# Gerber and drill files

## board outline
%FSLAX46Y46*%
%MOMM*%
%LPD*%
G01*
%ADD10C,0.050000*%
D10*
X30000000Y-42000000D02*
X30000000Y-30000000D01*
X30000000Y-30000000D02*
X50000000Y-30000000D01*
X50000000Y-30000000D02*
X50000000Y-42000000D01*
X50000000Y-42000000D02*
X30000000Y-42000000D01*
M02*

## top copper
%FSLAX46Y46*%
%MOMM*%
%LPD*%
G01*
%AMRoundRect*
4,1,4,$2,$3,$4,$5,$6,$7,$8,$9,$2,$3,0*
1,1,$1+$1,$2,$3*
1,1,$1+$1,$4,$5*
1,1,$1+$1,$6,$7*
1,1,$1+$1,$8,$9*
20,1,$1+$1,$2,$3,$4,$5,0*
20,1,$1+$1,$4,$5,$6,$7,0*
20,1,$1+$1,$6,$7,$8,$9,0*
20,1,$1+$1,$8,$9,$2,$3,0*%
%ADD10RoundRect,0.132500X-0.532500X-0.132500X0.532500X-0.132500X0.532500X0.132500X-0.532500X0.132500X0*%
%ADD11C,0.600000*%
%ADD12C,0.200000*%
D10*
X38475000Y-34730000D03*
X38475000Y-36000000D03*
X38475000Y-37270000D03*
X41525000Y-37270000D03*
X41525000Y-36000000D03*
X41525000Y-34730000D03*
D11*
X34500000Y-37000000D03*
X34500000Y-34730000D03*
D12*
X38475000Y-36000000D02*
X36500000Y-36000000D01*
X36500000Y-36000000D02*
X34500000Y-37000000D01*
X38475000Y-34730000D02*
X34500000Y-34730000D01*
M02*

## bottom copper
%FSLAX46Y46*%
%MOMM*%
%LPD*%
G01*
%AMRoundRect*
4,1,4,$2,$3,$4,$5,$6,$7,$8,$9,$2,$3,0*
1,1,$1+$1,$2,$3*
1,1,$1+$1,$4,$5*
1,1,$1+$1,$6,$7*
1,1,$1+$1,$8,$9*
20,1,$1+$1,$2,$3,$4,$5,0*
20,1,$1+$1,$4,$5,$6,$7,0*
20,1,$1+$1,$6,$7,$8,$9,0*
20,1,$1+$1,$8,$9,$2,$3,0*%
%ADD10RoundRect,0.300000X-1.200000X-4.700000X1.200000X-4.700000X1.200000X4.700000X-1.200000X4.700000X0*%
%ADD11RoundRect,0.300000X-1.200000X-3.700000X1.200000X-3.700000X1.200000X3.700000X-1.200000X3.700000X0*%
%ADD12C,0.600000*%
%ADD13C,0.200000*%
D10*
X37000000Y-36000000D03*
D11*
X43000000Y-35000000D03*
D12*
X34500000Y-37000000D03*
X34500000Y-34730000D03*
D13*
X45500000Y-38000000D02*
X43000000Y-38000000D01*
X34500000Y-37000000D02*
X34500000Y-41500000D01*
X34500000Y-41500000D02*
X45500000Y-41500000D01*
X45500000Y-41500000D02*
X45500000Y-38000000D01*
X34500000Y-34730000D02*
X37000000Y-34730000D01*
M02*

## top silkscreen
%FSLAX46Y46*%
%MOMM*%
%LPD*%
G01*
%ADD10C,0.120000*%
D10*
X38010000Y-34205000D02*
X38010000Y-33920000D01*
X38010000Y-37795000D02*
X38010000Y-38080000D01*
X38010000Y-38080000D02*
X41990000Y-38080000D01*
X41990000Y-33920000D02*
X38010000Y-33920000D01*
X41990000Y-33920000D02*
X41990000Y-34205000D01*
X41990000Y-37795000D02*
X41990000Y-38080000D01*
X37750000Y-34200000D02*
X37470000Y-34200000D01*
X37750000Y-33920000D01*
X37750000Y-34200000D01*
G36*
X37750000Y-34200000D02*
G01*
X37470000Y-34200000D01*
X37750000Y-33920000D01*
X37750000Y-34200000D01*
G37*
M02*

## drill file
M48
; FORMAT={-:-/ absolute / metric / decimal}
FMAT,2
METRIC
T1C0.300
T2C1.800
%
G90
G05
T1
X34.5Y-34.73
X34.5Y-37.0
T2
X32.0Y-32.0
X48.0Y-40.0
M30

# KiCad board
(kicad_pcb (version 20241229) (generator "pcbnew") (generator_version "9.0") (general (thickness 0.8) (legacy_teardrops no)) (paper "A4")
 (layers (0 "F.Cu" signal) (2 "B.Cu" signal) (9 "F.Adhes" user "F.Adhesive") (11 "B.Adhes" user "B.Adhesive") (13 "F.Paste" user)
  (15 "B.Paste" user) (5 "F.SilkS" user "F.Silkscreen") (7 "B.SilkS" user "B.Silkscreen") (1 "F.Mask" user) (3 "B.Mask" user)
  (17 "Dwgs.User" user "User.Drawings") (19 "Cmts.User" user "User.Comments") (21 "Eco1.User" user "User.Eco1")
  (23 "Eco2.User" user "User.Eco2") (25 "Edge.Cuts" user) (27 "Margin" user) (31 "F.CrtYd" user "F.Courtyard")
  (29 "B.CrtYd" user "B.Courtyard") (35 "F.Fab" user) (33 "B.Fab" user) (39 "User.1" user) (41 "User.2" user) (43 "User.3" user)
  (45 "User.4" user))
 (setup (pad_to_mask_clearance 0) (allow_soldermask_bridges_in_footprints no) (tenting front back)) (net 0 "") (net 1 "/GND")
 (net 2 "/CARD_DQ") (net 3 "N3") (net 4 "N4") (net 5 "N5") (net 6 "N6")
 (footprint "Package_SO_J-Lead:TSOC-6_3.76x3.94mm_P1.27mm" (layer "F.Cu") (at 40 36)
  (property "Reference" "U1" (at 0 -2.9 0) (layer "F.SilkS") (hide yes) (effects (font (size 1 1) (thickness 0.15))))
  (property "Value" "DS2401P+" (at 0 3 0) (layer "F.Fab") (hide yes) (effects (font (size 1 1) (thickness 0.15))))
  (fp_line (start -1.99 -1.795) (end -1.99 -2.08) (stroke (width 0.12) (type solid)) (layer "F.SilkS"))
  (fp_line (start -1.99 1.795) (end -1.99 2.08) (stroke (width 0.12) (type solid)) (layer "F.SilkS"))
  (fp_line (start -1.99 2.08) (end 1.99 2.08) (stroke (width 0.12) (type solid)) (layer "F.SilkS"))
  (fp_line (start 1.99 -2.08) (end -1.99 -2.08) (stroke (width 0.12) (type solid)) (layer "F.SilkS"))
  (fp_line (start 1.99 -2.08) (end 1.99 -1.795) (stroke (width 0.12) (type solid)) (layer "F.SilkS"))
  (fp_line (start 1.99 1.795) (end 1.99 2.08) (stroke (width 0.12) (type solid)) (layer "F.SilkS"))
  (fp_poly
   (pts (xy -2.25 -1.8) (xy -2.53 -1.8) (xy -2.25 -2.08) (xy -2.25 -1.8)) (stroke (width 0.12) (type solid)) (fill yes) (layer "F.SilkS"))
  (pad "1" smd roundrect (at -1.525 -1.27) (size 1.33 0.53) (layers "F.Cu" "F.Mask" "F.Paste") (roundrect_rratio 0.25) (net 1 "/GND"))
  (pad "2" smd roundrect (at -1.525 0) (size 1.33 0.53) (layers "F.Cu" "F.Mask" "F.Paste") (roundrect_rratio 0.25) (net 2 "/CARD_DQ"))
  (pad "3" smd roundrect (at -1.525 1.27) (size 1.33 0.53) (layers "F.Cu" "F.Mask" "F.Paste") (roundrect_rratio 0.25) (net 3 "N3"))
  (pad "4" smd roundrect (at 1.525 1.27) (size 1.33 0.53) (layers "F.Cu" "F.Mask" "F.Paste") (roundrect_rratio 0.25) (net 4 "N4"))
  (pad "5" smd roundrect (at 1.525 0) (size 1.33 0.53) (layers "F.Cu" "F.Mask" "F.Paste") (roundrect_rratio 0.25) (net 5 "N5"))
  (pad "6" smd roundrect (at 1.525 -1.27) (size 1.33 0.53) (layers "F.Cu" "F.Mask" "F.Paste") (roundrect_rratio 0.25) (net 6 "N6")))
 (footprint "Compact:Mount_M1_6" (layer "F.Cu") (at 32 32)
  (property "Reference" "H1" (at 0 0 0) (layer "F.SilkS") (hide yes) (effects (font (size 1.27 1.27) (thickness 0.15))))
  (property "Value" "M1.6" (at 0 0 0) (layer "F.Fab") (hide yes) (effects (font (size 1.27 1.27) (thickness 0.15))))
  (pad "" np_thru_hole circle (at 0 0) (size 1.8 1.8) (drill 1.8) (layers "*.Cu")))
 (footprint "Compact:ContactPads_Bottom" (layer "F.Cu") (at 30 30)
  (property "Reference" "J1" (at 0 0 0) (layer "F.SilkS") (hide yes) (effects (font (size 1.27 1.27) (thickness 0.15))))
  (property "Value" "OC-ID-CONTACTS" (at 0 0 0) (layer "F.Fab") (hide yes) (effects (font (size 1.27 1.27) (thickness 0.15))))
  (pad "1" smd roundrect (at 7 6) (size 3 10) (layers "B.Cu" "B.Mask") (roundrect_rratio 0.1) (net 1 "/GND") (thermal_bridge_angle 45))
  (pad "2" smd roundrect (at 13 5) (size 3 8) (layers "B.Cu" "B.Mask") (roundrect_rratio 0.1) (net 2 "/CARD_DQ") (thermal_bridge_angle 45)))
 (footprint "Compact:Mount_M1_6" (layer "F.Cu") (at 48 40)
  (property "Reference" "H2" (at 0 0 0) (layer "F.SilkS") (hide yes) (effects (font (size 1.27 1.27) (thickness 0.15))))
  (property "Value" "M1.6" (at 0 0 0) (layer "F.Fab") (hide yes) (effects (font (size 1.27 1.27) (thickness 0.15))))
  (pad "" np_thru_hole circle (at 0 0) (size 1.8 1.8) (drill 1.8) (layers "*.Cu")))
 (gr_line (start 30 42) (end 30 30) (stroke (width 0.05) (type default)) (layer "Edge.Cuts"))
 (gr_line (start 30 30) (end 50 30) (stroke (width 0.05) (type default)) (layer "Edge.Cuts"))
 (gr_line (start 50 30) (end 50 42) (stroke (width 0.05) (type default)) (layer "Edge.Cuts"))
 (gr_line (start 50 42) (end 30 42) (stroke (width 0.05) (type default)) (layer "Edge.Cuts"))
 (segment (start 38.475 36) (end 36.5 36) (width 0.2) (layer "F.Cu") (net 2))
 (segment (start 36.5 36) (end 34.5 37) (width 0.2) (layer "F.Cu") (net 2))
 (via (at 34.5 37) (size 0.6) (drill 0.3) (layers "F.Cu" "B.Cu") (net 2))
 (segment (start 45.5 38) (end 43 38) (width 0.2) (layer "B.Cu") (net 2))
 (segment (start 34.5 37) (end 34.5 41.5) (width 0.2) (layer "B.Cu") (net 2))
 (segment (start 34.5 41.5) (end 45.5 41.5) (width 0.2) (layer "B.Cu") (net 2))
 (segment (start 45.5 41.5) (end 45.5 38) (width 0.2) (layer "B.Cu") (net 2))
 (segment (start 38.475 34.73) (end 34.5 34.73) (width 0.2) (layer "F.Cu") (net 1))
 (via (at 34.5 34.73) (size 0.6) (drill 0.3) (layers "F.Cu" "B.Cu") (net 1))
 (segment (start 34.5 34.73) (end 37 34.73) (width 0.2) (layer "B.Cu") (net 1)))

